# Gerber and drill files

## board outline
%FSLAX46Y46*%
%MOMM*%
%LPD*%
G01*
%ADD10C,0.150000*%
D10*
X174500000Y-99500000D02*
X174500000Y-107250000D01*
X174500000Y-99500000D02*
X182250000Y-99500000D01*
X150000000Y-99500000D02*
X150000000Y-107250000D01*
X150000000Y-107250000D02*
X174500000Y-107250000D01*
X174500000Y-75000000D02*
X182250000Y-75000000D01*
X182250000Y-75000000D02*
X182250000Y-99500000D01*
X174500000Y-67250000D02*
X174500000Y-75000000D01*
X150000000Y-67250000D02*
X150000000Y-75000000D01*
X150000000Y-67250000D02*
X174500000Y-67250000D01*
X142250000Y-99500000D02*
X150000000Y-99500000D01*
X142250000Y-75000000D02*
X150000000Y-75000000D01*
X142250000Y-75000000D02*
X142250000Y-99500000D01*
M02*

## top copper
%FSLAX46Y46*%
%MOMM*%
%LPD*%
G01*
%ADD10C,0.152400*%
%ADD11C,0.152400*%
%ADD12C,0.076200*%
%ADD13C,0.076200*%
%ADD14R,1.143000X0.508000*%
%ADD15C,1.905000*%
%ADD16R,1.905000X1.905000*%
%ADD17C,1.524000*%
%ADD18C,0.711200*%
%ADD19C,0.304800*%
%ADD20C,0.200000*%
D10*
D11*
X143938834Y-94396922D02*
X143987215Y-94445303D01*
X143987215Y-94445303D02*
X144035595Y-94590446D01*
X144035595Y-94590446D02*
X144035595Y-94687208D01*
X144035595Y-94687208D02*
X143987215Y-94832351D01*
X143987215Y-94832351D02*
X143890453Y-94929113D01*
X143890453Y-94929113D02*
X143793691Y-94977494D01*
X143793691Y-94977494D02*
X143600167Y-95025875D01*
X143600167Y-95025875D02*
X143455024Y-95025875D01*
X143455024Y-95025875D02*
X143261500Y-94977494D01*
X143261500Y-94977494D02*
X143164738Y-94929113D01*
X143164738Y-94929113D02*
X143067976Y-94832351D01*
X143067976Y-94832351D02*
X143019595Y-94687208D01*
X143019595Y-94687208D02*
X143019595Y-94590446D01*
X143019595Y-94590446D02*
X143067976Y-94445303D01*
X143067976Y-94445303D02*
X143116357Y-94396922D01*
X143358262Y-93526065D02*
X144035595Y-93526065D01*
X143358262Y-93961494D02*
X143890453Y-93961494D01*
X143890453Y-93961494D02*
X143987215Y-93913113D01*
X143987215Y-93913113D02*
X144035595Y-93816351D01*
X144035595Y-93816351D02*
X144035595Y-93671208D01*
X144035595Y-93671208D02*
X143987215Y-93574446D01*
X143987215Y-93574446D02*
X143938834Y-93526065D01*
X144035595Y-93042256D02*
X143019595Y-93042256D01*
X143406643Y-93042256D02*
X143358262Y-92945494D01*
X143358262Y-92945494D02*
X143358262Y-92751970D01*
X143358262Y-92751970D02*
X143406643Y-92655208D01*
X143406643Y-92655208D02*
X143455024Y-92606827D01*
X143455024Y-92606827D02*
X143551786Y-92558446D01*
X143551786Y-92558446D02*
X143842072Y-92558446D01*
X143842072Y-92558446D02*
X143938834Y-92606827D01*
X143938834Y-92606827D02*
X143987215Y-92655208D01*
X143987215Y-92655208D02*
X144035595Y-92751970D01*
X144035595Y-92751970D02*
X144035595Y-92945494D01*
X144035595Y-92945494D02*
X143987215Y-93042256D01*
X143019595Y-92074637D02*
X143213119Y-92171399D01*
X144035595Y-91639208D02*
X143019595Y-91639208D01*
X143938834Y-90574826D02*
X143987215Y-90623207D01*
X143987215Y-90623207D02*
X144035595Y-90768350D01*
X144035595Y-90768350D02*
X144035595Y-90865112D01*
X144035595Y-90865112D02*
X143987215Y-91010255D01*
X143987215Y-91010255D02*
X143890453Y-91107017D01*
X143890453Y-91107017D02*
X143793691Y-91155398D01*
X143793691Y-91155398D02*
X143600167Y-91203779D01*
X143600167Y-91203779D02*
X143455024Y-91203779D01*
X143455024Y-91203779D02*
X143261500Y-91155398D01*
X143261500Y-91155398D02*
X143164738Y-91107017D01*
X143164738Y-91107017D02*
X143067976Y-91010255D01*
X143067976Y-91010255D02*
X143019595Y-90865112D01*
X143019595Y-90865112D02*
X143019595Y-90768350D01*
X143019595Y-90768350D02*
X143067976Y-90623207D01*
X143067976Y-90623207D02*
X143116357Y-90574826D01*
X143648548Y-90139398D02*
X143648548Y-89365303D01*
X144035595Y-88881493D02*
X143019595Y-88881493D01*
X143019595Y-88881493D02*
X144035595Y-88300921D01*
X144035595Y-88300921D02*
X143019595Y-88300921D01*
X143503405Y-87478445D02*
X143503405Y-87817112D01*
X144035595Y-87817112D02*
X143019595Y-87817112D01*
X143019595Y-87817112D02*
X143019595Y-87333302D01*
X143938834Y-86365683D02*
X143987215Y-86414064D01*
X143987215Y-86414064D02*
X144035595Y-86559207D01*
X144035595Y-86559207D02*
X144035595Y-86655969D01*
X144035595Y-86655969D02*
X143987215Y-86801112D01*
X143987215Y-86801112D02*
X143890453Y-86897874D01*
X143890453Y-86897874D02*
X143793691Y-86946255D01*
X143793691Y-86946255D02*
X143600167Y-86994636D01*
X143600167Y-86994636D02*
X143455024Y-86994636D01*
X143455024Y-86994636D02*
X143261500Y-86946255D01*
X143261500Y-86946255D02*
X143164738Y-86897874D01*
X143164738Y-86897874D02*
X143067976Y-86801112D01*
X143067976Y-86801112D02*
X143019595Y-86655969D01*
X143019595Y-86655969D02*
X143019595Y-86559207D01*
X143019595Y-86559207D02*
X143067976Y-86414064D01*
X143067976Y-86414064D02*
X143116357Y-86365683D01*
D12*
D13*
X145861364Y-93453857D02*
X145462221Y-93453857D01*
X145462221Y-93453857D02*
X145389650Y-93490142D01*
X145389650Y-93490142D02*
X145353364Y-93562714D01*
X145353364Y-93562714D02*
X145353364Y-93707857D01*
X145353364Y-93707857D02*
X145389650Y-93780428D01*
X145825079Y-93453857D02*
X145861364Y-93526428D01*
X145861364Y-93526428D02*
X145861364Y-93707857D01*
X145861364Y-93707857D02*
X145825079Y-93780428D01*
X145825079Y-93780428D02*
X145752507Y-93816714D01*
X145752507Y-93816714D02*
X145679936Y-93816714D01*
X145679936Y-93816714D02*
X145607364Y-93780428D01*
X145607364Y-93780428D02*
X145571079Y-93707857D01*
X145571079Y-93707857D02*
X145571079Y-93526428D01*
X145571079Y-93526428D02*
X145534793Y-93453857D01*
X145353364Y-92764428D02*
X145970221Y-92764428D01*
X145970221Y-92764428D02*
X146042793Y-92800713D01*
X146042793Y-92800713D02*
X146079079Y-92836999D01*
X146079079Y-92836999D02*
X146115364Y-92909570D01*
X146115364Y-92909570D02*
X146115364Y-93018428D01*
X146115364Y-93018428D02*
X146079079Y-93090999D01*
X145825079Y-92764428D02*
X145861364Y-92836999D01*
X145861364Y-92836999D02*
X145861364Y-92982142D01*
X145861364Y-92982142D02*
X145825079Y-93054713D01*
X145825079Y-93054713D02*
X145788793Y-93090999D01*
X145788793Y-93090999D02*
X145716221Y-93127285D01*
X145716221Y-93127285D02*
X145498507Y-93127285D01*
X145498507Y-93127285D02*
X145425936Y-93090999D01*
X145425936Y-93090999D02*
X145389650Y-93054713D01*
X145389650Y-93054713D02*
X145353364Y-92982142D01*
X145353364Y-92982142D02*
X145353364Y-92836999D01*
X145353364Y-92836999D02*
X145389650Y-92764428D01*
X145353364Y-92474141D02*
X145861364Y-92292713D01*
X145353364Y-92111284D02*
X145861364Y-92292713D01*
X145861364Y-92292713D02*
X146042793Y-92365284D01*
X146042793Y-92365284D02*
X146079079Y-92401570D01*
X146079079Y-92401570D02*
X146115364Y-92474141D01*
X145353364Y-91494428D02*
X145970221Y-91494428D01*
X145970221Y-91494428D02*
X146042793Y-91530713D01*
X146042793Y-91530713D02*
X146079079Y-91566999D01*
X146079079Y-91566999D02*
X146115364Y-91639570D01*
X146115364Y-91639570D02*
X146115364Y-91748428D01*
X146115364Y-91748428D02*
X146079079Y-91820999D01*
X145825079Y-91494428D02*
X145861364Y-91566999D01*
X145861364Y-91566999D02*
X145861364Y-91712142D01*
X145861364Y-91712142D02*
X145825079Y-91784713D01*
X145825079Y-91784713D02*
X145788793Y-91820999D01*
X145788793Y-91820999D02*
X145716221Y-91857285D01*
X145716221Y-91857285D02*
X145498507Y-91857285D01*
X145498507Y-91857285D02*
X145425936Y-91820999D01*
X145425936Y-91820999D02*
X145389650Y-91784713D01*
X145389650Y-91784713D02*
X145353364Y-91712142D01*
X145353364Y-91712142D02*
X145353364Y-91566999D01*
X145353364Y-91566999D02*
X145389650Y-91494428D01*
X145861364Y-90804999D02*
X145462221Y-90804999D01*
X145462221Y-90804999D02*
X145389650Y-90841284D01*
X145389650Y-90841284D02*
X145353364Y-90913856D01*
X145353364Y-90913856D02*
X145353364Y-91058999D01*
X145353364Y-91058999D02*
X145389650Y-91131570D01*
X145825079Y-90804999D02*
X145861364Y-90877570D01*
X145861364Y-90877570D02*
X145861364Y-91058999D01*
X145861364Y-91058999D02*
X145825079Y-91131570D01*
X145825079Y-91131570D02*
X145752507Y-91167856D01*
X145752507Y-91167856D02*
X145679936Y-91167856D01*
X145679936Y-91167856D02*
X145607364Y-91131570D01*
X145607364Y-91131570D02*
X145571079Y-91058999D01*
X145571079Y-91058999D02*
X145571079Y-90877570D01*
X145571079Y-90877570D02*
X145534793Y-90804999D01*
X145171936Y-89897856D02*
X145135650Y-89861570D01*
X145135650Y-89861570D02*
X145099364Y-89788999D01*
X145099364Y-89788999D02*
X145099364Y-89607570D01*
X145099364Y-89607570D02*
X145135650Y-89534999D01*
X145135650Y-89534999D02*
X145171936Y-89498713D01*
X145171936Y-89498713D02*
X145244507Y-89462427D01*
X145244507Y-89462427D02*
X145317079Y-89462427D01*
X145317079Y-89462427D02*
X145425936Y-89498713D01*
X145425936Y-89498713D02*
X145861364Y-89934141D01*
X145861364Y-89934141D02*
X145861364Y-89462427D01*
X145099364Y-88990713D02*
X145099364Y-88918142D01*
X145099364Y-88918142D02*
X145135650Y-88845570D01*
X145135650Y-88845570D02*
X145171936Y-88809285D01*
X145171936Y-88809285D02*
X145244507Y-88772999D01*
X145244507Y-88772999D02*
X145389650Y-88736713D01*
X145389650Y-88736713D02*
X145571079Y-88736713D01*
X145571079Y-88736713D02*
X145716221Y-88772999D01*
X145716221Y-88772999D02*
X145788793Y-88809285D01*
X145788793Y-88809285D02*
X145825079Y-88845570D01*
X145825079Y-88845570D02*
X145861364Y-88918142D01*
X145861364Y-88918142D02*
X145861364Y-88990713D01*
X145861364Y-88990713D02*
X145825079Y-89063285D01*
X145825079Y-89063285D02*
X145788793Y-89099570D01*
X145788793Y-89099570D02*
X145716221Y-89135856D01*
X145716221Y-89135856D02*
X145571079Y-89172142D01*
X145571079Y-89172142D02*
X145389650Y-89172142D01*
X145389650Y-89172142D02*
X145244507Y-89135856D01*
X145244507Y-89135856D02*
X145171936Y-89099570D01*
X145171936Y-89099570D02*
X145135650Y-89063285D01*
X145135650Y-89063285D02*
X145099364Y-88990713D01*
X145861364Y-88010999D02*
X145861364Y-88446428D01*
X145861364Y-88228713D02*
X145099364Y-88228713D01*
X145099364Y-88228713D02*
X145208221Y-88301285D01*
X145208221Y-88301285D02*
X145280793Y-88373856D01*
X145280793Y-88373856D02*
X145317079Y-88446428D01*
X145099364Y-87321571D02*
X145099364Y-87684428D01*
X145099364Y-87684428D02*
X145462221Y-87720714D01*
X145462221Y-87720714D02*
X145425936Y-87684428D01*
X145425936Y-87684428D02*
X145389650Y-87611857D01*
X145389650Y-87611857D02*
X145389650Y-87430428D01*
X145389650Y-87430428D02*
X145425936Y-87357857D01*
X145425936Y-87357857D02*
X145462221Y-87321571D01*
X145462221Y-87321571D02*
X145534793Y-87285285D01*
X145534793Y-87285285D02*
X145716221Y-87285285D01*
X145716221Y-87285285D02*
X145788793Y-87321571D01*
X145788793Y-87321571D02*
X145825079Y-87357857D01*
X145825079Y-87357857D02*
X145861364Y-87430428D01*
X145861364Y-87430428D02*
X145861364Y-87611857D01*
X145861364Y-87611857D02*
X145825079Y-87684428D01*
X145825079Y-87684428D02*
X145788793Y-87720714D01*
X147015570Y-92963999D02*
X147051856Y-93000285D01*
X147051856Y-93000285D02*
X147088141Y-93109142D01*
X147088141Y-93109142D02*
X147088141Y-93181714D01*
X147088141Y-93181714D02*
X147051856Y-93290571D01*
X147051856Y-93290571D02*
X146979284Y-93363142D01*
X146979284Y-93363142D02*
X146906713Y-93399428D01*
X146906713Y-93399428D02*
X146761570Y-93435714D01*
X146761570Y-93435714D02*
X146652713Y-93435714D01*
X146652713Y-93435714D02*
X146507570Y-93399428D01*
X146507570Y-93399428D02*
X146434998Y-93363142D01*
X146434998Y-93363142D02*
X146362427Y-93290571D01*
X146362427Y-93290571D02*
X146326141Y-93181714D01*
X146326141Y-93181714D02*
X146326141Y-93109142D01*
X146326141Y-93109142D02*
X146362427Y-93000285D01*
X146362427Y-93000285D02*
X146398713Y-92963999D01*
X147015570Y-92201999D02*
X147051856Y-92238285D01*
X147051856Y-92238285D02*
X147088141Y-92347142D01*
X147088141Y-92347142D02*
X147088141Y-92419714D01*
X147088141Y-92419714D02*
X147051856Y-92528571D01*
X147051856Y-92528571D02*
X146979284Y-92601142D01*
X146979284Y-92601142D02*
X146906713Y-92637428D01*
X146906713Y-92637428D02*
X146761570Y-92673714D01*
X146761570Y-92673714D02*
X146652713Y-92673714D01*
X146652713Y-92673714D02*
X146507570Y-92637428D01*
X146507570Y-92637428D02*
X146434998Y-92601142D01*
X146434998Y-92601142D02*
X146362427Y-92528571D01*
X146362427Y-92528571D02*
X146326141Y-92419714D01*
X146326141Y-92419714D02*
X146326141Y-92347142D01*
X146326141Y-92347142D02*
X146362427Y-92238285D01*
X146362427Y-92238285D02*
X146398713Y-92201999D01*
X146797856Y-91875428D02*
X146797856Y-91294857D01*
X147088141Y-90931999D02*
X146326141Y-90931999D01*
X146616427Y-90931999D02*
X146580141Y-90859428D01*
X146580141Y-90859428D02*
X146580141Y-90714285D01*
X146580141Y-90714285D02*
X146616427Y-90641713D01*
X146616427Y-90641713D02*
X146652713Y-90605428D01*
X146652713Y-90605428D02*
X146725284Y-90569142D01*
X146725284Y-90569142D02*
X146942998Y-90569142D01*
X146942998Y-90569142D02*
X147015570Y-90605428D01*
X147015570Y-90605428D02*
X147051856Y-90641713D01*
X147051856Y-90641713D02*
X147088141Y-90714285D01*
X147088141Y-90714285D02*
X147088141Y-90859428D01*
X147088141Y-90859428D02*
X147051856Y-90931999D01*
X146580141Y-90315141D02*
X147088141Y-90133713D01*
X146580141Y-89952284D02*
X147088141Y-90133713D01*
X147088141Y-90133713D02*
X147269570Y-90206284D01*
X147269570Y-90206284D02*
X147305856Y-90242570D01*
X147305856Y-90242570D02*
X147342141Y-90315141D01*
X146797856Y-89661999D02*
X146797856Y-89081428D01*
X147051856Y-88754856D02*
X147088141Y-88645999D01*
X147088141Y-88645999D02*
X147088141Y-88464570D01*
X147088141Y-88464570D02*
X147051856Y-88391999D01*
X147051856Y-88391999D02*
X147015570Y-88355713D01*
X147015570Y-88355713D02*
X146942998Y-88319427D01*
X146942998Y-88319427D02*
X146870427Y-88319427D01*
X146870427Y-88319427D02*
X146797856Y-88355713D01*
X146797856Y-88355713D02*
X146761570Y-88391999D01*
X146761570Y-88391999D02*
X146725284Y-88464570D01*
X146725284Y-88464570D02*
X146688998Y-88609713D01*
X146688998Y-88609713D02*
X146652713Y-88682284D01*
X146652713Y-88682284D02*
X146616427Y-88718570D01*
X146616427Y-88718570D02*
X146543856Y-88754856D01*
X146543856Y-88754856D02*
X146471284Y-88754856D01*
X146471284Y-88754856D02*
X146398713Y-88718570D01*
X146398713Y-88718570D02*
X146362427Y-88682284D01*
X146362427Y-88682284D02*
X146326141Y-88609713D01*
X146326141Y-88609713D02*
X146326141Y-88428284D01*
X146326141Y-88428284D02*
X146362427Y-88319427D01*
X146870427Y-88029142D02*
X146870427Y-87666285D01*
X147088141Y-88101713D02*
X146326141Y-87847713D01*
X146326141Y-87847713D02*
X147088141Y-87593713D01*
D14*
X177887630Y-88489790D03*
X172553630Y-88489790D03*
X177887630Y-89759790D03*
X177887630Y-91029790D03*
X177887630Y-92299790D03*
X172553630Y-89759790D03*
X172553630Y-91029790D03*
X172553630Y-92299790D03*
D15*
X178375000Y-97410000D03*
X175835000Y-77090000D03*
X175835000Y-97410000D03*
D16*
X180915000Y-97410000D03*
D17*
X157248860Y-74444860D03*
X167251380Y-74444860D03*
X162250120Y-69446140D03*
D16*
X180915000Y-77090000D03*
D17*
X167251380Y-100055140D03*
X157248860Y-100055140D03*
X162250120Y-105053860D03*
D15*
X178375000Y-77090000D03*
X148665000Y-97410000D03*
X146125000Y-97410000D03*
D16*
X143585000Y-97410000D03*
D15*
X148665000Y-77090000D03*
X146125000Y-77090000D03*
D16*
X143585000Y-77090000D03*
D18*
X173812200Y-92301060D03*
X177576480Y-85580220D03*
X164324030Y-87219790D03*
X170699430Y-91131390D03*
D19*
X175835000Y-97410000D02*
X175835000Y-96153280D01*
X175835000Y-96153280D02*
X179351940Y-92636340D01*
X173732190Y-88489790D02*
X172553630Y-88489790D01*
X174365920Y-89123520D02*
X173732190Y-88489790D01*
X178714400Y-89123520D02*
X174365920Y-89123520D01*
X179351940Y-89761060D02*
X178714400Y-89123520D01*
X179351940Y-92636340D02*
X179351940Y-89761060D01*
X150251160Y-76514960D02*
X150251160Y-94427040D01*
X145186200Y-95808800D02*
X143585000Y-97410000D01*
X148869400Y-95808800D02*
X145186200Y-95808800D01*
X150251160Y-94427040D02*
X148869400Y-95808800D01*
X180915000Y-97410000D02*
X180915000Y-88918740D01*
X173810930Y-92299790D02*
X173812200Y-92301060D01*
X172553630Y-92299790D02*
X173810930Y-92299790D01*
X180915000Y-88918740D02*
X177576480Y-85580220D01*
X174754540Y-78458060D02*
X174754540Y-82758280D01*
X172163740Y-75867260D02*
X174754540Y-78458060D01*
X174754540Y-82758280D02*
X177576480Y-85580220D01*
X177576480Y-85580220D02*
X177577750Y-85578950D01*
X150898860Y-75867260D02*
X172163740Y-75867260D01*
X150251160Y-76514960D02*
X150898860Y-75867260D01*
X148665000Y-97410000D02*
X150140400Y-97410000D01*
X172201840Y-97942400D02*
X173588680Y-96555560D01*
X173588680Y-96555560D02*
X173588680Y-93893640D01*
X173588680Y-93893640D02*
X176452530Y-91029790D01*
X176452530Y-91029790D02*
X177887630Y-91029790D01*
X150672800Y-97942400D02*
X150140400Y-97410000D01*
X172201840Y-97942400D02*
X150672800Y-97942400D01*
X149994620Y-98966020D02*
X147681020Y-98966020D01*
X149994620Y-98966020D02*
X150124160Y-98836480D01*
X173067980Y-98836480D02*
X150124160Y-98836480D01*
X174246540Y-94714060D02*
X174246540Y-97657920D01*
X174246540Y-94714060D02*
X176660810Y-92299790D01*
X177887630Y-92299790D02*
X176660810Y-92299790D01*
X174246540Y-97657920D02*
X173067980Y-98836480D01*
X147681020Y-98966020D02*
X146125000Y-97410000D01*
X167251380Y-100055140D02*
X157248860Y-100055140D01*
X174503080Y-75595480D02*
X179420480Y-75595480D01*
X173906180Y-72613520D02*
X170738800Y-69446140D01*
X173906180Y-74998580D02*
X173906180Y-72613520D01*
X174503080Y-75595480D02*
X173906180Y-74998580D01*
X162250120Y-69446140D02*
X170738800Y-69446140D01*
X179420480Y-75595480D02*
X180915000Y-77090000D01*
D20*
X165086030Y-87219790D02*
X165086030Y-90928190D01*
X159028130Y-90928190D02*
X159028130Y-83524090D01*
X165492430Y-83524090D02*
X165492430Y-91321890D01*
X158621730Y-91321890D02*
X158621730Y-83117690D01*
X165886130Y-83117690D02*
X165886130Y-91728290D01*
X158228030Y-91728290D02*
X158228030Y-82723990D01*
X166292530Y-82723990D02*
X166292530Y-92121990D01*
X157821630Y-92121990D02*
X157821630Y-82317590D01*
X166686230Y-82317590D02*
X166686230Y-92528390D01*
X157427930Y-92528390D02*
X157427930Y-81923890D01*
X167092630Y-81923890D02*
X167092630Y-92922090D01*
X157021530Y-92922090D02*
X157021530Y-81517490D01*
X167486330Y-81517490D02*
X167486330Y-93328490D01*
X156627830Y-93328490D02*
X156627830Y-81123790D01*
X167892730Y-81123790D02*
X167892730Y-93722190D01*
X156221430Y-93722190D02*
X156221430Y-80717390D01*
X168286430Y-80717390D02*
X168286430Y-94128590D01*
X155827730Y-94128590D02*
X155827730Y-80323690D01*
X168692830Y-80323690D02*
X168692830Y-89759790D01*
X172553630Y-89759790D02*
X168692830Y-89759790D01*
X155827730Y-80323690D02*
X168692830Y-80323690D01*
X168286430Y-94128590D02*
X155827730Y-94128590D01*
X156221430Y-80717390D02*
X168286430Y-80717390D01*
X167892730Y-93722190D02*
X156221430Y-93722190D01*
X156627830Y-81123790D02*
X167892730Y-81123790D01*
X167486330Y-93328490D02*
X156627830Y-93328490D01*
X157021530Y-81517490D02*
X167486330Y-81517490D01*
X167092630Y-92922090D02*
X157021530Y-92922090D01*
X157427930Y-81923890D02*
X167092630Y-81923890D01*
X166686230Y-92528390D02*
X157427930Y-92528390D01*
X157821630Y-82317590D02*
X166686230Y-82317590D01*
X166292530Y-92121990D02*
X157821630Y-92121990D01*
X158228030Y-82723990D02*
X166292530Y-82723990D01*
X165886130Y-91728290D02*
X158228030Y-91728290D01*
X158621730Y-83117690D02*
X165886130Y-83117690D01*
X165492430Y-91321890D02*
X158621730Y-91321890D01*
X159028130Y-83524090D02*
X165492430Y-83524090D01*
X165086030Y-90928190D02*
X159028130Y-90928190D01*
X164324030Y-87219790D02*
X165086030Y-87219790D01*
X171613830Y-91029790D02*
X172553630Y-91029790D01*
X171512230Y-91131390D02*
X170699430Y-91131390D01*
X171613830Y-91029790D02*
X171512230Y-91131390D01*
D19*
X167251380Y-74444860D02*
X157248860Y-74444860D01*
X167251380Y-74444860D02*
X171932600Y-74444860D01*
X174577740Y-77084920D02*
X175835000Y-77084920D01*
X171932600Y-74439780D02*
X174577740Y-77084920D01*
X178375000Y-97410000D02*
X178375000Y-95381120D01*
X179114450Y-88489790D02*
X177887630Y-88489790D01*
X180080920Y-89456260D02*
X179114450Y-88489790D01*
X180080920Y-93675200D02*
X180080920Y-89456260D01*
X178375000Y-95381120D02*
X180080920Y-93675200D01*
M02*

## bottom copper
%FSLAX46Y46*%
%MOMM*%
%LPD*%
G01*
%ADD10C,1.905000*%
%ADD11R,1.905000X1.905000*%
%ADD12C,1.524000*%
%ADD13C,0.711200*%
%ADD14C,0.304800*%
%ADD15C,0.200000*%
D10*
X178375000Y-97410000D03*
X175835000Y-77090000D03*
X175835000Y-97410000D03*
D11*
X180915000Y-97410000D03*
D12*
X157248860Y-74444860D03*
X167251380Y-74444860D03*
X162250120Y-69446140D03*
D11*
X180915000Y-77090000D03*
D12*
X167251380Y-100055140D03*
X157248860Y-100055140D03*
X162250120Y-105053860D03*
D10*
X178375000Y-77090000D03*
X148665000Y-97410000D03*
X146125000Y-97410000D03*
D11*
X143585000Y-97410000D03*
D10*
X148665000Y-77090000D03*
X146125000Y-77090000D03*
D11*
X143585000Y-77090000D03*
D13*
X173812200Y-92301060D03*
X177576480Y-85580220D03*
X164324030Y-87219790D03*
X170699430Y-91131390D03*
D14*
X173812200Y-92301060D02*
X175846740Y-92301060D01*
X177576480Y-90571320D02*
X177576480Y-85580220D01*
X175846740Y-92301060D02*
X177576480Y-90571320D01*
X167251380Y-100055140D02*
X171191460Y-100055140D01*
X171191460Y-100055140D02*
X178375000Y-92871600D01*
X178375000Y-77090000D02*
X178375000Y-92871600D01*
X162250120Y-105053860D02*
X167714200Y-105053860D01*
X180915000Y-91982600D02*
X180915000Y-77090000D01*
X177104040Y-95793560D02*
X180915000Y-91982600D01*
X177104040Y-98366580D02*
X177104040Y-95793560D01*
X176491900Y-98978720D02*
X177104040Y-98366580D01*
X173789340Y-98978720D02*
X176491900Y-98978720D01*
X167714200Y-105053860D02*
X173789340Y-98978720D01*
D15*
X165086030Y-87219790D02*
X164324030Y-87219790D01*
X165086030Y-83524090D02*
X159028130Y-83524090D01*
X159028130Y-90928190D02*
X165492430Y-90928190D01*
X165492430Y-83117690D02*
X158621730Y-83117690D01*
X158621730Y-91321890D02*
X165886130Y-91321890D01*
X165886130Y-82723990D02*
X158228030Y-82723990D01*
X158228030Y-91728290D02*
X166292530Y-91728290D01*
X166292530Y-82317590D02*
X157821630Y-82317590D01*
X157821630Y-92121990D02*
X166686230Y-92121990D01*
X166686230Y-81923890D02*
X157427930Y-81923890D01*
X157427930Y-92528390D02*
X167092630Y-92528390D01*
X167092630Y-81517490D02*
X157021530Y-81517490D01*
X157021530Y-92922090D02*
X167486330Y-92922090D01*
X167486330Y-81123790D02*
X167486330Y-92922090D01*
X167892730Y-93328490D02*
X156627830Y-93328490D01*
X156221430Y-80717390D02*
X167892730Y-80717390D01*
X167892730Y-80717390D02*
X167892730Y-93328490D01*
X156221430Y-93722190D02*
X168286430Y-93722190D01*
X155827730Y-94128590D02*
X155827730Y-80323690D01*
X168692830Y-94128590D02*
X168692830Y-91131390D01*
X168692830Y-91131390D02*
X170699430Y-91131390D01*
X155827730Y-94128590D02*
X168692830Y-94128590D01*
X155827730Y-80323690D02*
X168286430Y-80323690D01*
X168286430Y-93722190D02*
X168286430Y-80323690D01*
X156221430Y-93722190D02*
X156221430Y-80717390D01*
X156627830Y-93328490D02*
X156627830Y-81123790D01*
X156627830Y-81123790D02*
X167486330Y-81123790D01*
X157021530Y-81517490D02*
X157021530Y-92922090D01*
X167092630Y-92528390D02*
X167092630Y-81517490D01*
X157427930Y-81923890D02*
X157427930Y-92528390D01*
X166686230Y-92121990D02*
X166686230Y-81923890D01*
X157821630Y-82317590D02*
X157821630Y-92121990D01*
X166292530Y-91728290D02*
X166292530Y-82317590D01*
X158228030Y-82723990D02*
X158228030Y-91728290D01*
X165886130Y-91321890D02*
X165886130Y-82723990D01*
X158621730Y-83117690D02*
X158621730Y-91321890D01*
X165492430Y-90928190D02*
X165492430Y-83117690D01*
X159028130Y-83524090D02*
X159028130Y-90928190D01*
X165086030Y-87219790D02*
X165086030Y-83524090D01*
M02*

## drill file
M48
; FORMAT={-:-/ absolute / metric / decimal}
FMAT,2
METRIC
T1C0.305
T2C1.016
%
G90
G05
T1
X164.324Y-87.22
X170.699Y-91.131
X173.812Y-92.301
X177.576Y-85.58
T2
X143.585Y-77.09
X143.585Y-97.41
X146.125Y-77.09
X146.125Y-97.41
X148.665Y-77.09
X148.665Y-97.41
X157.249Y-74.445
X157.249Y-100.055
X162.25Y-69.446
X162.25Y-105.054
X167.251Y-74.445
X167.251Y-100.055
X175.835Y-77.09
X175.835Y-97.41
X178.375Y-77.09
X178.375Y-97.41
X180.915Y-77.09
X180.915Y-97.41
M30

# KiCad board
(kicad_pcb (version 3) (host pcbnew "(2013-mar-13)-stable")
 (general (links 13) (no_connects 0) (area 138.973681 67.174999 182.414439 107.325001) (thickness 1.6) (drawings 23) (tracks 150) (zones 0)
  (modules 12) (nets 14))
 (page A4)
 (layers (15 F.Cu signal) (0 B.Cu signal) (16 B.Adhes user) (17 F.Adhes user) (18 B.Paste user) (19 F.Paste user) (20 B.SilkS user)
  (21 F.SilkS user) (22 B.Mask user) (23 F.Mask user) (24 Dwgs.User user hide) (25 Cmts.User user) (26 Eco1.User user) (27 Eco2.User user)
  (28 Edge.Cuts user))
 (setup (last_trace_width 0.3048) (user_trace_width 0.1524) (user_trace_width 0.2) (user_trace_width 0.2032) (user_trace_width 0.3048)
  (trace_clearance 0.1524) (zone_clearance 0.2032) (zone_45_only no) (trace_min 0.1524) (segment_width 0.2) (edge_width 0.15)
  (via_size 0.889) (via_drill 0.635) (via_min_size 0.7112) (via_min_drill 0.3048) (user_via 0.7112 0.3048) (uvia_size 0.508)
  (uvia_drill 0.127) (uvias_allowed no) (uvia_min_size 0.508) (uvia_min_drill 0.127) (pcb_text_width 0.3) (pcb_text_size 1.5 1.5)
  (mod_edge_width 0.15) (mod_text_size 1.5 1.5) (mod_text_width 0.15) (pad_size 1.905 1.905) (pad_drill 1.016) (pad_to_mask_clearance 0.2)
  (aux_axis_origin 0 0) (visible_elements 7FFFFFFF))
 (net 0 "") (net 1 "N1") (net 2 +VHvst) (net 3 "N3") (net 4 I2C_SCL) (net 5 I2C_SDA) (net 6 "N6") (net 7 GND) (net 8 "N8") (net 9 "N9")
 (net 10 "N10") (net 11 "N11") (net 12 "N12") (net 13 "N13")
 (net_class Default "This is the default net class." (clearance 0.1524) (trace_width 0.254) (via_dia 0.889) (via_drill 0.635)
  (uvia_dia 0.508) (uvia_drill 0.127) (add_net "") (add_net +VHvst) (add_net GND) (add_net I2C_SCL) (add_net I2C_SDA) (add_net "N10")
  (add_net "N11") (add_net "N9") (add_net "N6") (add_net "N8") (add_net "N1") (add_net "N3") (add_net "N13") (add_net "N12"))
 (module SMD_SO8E (layer F.Cu) (at 175.22063 90.39479 270)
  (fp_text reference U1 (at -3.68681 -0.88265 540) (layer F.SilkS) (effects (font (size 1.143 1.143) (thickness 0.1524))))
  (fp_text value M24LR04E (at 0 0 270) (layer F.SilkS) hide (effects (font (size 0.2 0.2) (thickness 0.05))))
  (pad 8 smd rect (at -1.905 -2.667 270) (size 0.508 1.143) (layers F.Cu F.Paste F.Mask) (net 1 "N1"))
  (pad 1 smd rect (at -1.905 2.667 270) (size 0.508 1.143) (layers F.Cu F.Paste F.Mask) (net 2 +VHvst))
  (pad 7 smd rect (at -0.635 -2.667 270) (size 0.508 1.143) (layers F.Cu F.Paste F.Mask) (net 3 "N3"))
  (pad 6 smd rect (at 0.635 -2.667 270) (size 0.508 1.143) (layers F.Cu F.Paste F.Mask) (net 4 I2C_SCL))
  (pad 5 smd rect (at 1.905 -2.667 270) (size 0.508 1.143) (layers F.Cu F.Paste F.Mask) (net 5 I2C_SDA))
  (pad 2 smd rect (at -0.635 2.667 270) (size 0.508 1.143) (layers F.Cu F.Paste F.Mask) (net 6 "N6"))
  (pad 3 smd rect (at 0.635 2.667 270) (size 0.508 1.143) (layers F.Cu F.Paste F.Mask) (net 6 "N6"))
  (pad 4 smd rect (at 1.905 2.667 270) (size 0.508 1.143) (layers F.Cu F.Paste F.Mask) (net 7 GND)))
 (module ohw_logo (layer F.Cu) (at 142.27048 78.73492)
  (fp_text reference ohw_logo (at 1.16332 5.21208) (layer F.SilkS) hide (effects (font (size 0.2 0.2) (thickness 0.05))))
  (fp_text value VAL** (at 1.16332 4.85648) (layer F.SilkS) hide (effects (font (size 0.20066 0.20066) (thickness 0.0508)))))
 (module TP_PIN (layer F.Cu) (at 178.375 97.41)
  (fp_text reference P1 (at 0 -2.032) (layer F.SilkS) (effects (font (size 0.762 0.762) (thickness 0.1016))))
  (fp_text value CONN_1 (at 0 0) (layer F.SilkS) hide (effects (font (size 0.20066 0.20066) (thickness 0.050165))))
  (pad 1 thru_hole circle (at 0 0) (size 1.905 1.905) (drill 1.016) (layers *.Cu *.Mask F.SilkS) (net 1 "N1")))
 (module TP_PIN (layer F.Cu) (at 175.835 77.09)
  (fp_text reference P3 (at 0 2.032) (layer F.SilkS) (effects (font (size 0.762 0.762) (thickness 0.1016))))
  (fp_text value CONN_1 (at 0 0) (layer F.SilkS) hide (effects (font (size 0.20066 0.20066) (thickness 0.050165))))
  (pad 1 thru_hole circle (at 0 0) (size 1.905 1.905) (drill 1.016) (layers *.Cu *.Mask F.SilkS) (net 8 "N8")))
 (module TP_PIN (layer F.Cu) (at 175.835 97.41)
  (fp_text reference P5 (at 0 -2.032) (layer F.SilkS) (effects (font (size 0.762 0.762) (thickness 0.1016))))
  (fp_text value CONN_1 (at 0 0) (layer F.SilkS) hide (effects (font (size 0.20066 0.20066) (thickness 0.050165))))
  (pad 1 thru_hole circle (at 0 0) (size 1.905 1.905) (drill 1.016) (layers *.Cu *.Mask F.SilkS) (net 2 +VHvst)))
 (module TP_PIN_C (layer F.Cu) (at 180.915 97.41)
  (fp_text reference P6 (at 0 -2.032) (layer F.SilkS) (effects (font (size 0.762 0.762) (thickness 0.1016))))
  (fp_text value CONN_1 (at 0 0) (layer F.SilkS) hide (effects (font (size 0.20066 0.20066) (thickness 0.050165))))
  (pad 1 thru_hole rect (at 0 0) (size 1.905 1.905) (drill 1.016) (layers *.Cu *.Mask F.SilkS) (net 7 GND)))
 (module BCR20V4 (layer F.Cu) (at 162.25012 71.9455)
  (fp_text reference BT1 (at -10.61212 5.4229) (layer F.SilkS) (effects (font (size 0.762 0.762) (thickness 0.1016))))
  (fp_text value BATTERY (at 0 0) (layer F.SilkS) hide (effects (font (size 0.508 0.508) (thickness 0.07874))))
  (pad 1 thru_hole circle (at -5.00126 2.49936) (size 1.524 1.524) (drill 1.016) (layers *.Cu *.Mask) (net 8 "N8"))
  (pad 1 thru_hole circle (at 5.00126 2.49936) (size 1.524 1.524) (drill 1.016) (layers *.Cu *.Mask) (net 8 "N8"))
  (pad 2 thru_hole circle (at 0 -2.49936) (size 1.524 1.524) (drill 1.016) (layers *.Cu *.Mask) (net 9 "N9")))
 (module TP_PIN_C (layer F.Cu) (at 180.915 77.09)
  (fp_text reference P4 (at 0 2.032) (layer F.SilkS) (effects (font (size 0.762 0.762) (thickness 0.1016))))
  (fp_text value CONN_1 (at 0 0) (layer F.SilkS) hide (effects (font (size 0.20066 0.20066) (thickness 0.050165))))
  (pad 1 thru_hole rect (at 0 0) (size 1.905 1.905) (drill 1.016) (layers *.Cu *.Mask F.SilkS) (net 9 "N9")))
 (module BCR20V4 (layer F.Cu) (at 162.25012 102.5545 180)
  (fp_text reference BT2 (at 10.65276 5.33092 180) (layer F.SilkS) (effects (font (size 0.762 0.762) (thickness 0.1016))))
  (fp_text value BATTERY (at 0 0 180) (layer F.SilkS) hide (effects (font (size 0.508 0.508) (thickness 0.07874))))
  (pad 1 thru_hole circle (at -5.00126 2.49936 180) (size 1.524 1.524) (drill 1.016) (layers *.Cu *.Mask) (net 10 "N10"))
  (pad 1 thru_hole circle (at 5.00126 2.49936 180) (size 1.524 1.524) (drill 1.016) (layers *.Cu *.Mask) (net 10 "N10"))
  (pad 2 thru_hole circle (at 0 -2.49936 180) (size 1.524 1.524) (drill 1.016) (layers *.Cu *.Mask) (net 9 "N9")))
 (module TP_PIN (layer F.Cu) (at 178.375 77.09)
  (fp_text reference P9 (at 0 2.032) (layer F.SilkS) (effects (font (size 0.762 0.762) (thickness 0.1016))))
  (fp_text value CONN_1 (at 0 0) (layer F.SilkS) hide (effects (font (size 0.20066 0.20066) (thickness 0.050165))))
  (pad 1 thru_hole circle (at 0 0) (size 1.905 1.905) (drill 1.016) (layers *.Cu *.Mask F.SilkS) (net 10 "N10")))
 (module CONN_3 (layer F.Cu) (at 146.125 97.41)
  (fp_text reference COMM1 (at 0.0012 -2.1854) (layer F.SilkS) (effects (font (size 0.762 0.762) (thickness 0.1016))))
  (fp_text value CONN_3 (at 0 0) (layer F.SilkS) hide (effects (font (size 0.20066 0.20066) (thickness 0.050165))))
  (pad 3 thru_hole circle (at 2.54 0) (size 1.905 1.905) (drill 1.016) (layers *.Cu *.Mask F.SilkS) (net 4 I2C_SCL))
  (pad 2 thru_hole circle (at 0 0) (size 1.905 1.905) (drill 1.016) (layers *.Cu *.Mask F.SilkS) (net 5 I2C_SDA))
  (pad 1 thru_hole rect (at -2.54 0) (size 1.905 1.905) (drill 1.016) (layers *.Cu *.Mask F.SilkS) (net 7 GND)))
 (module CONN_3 (layer F.Cu) (at 146.125 77.09)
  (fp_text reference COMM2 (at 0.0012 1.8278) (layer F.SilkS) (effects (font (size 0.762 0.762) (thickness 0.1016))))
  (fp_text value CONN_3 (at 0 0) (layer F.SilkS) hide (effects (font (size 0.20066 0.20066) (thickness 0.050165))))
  (pad 3 thru_hole circle (at 2.54 0) (size 1.905 1.905) (drill 1.016) (layers *.Cu *.Mask F.SilkS) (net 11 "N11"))
  (pad 2 thru_hole circle (at 0 0) (size 1.905 1.905) (drill 1.016) (layers *.Cu *.Mask F.SilkS) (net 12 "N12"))
  (pad 1 thru_hole rect (at -2.54 0) (size 1.905 1.905) (drill 1.016) (layers *.Cu *.Mask F.SilkS) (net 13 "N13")))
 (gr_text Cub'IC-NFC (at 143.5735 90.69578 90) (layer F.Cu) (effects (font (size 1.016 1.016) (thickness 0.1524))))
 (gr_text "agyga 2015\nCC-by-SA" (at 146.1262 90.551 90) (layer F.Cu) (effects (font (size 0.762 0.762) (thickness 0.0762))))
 (gr_line (start 174.5 99.5) (end 174.5 107.25) (angle 90) (layer Edge.Cuts) (width 0.15))
 (gr_line (start 174.5 99.5) (end 182.25 99.5) (angle 90) (layer Edge.Cuts) (width 0.15))
 (gr_line (start 150 99.5) (end 150 107.25) (angle 90) (layer Edge.Cuts) (width 0.15))
 (gr_line (start 150 107.25) (end 174.5 107.25) (angle 90) (layer Edge.Cuts) (width 0.15))
 (gr_line (start 174.5 75) (end 182.25 75) (angle 90) (layer Edge.Cuts) (width 0.15))
 (gr_line (start 182.25 75) (end 182.25 99.5) (angle 90) (layer Edge.Cuts) (width 0.15))
 (gr_line (start 174.5 67.25) (end 174.5 75) (angle 90) (layer Edge.Cuts) (width 0.15))
 (gr_line (start 150 67.25) (end 150 75) (angle 90) (layer Edge.Cuts) (width 0.15))
 (gr_line (start 150 67.25) (end 174.5 67.25) (angle 90) (layer Edge.Cuts) (width 0.15))
 (gr_line (start 142.25 99.5) (end 150 99.5) (angle 90) (layer Edge.Cuts) (width 0.15))
 (gr_line (start 142.25 75) (end 150 75) (angle 90) (layer Edge.Cuts) (width 0.15))
 (gr_line (start 142.25 75) (end 142.25 99.5) (angle 90) (layer Edge.Cuts) (width 0.15))
 (segment (start 175.835 97.41) (end 175.835 96.15328) (width 0.3048) (layer F.Cu) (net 2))
 (segment (start 175.835 96.15328) (end 179.35194 92.63634) (width 0.3048) (layer F.Cu) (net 2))
 (segment (start 173.73219 88.48979) (end 172.55363 88.48979) (width 0.3048) (layer F.Cu) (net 2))
 (segment (start 174.36592 89.12352) (end 173.73219 88.48979) (width 0.3048) (layer F.Cu) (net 2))
 (segment (start 178.7144 89.12352) (end 174.36592 89.12352) (width 0.3048) (layer F.Cu) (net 2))
 (segment (start 179.35194 89.76106) (end 178.7144 89.12352) (width 0.3048) (layer F.Cu) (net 2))
 (segment (start 179.35194 92.63634) (end 179.35194 89.76106) (width 0.3048) (layer F.Cu) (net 2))
 (segment (start 150.25116 76.51496) (end 150.25116 94.42704) (width 0.3048) (layer F.Cu) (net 7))
 (segment (start 145.1862 95.8088) (end 143.585 97.41) (width 0.3048) (layer F.Cu) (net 7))
 (segment (start 148.8694 95.8088) (end 145.1862 95.8088) (width 0.3048) (layer F.Cu) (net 7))
 (segment (start 150.25116 94.42704) (end 148.8694 95.8088) (width 0.3048) (layer F.Cu) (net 7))
 (segment (start 180.915 97.41) (end 180.915 88.91874) (width 0.3048) (layer F.Cu) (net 7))
 (segment (start 173.8122 92.30106) (end 175.84674 92.30106) (width 0.3048) (layer B.Cu) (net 7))
 (segment (start 173.81093 92.29979) (end 173.8122 92.30106) (width 0.3048) (layer F.Cu) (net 7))
 (via (at 173.8122 92.30106) (size 0.7112) (drill 0.3048) (layers F.Cu B.Cu) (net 7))
 (segment (start 172.55363 92.29979) (end 173.81093 92.29979) (width 0.3048) (layer F.Cu) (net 7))
 (segment (start 180.915 88.91874) (end 177.57648 85.58022) (width 0.3048) (layer F.Cu) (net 7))
 (segment (start 174.75454 78.45806) (end 174.75454 82.75828) (width 0.3048) (layer F.Cu) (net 7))
 (segment (start 172.16374 75.86726) (end 174.75454 78.45806) (width 0.3048) (layer F.Cu) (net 7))
 (segment (start 174.75454 82.75828) (end 177.57648 85.58022) (width 0.3048) (layer F.Cu) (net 7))
 (segment (start 177.57648 85.58022) (end 177.57775 85.57895) (width 0.3048) (layer F.Cu) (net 7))
 (via (at 177.57648 85.58022) (size 0.7112) (drill 0.3048) (layers F.Cu B.Cu) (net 7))
 (segment (start 177.57648 90.57132) (end 177.57648 85.58022) (width 0.3048) (layer B.Cu) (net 7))
 (segment (start 175.84674 92.30106) (end 177.57648 90.57132) (width 0.3048) (layer B.Cu) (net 7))
 (segment (start 150.89886 75.86726) (end 172.16374 75.86726) (width 0.3048) (layer F.Cu) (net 7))
 (segment (start 150.25116 76.51496) (end 150.89886 75.86726) (width 0.3048) (layer F.Cu) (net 7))
 (segment (start 148.665 97.41) (end 150.1404 97.41) (width 0.3048) (layer F.Cu) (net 4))
 (segment (start 172.20184 97.9424) (end 173.58868 96.55556) (width 0.3048) (layer F.Cu) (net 4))
 (segment (start 173.58868 96.55556) (end 173.58868 93.89364) (width 0.3048) (layer F.Cu) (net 4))
 (segment (start 173.58868 93.89364) (end 176.45253 91.02979) (width 0.3048) (layer F.Cu) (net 4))
 (segment (start 176.45253 91.02979) (end 177.88763 91.02979) (width 0.3048) (layer F.Cu) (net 4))
 (segment (start 150.6728 97.9424) (end 150.1404 97.41) (width 0.3048) (layer F.Cu) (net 4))
 (segment (start 172.20184 97.9424) (end 150.6728 97.9424) (width 0.3048) (layer F.Cu) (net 4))
 (segment (start 149.99462 98.96602) (end 147.68102 98.96602) (width 0.3048) (layer F.Cu) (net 5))
 (segment (start 149.99462 98.96602) (end 150.12416 98.83648) (width 0.3048) (layer F.Cu) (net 5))
 (segment (start 173.06798 98.83648) (end 150.12416 98.83648) (width 0.3048) (layer F.Cu) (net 5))
 (segment (start 174.24654 94.71406) (end 174.24654 97.65792) (width 0.3048) (layer F.Cu) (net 5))
 (segment (start 174.24654 94.71406) (end 176.66081 92.29979) (width 0.3048) (layer F.Cu) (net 5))
 (segment (start 177.88763 92.29979) (end 176.66081 92.29979) (width 0.3048) (layer F.Cu) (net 5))
 (segment (start 174.24654 97.65792) (end 173.06798 98.83648) (width 0.3048) (layer F.Cu) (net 5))
 (segment (start 147.68102 98.96602) (end 146.125 97.41) (width 0.3048) (layer F.Cu) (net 5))
 (segment (start 167.25138 100.05514) (end 171.19146 100.05514) (width 0.3048) (layer B.Cu) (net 10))
 (segment (start 171.19146 100.05514) (end 178.375 92.8716) (width 0.3048) (layer B.Cu) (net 10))
 (segment (start 167.25138 100.05514) (end 157.24886 100.05514) (width 0.3048) (layer F.Cu) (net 10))
 (segment (start 178.375 77.09) (end 178.375 92.8716) (width 0.3048) (layer B.Cu) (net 10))
 (segment (start 162.25012 105.05386) (end 167.7142 105.05386) (width 0.3048) (layer B.Cu) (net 9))
 (segment (start 180.915 91.9826) (end 180.915 77.09) (width 0.3048) (layer B.Cu) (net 9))
 (segment (start 177.10404 95.79356) (end 180.915 91.9826) (width 0.3048) (layer B.Cu) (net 9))
 (segment (start 177.10404 98.36658) (end 177.10404 95.79356) (width 0.3048) (layer B.Cu) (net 9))
 (segment (start 176.4919 98.97872) (end 177.10404 98.36658) (width 0.3048) (layer B.Cu) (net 9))
 (segment (start 173.78934 98.97872) (end 176.4919 98.97872) (width 0.3048) (layer B.Cu) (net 9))
 (segment (start 167.7142 105.05386) (end 173.78934 98.97872) (width 0.3048) (layer B.Cu) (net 9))
 (segment (start 174.50308 75.59548) (end 179.42048 75.59548) (width 0.3048) (layer F.Cu) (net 9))
 (segment (start 173.90618 72.61352) (end 170.7388 69.44614) (width 0.3048) (layer F.Cu) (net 9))
 (segment (start 173.90618 74.99858) (end 173.90618 72.61352) (width 0.3048) (layer F.Cu) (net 9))
 (segment (start 174.50308 75.59548) (end 173.90618 74.99858) (width 0.3048) (layer F.Cu) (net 9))
 (segment (start 162.25012 69.44614) (end 170.7388 69.44614) (width 0.3048) (layer F.Cu) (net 9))
 (segment (start 179.42048 75.59548) (end 180.915 77.09) (width 0.3048) (layer F.Cu) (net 9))
 (segment (start 165.08603 87.21979) (end 164.32403 87.21979) (width 0.2) (layer B.Cu) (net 6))
 (via (at 164.32403 87.21979) (size 0.7112) (drill 0.3048) (layers F.Cu B.Cu) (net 6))
 (segment (start 165.08603 87.21979) (end 165.08603 90.92819) (width 0.2) (layer F.Cu) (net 6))
 (segment (start 159.02813 90.92819) (end 159.02813 83.52409) (width 0.2) (layer F.Cu) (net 6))
 (segment (start 165.49243 83.52409) (end 165.49243 91.32189) (width 0.2) (layer F.Cu) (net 6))
 (segment (start 158.62173 91.32189) (end 158.62173 83.11769) (width 0.2) (layer F.Cu) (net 6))
 (segment (start 165.88613 83.11769) (end 165.88613 91.72829) (width 0.2) (layer F.Cu) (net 6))
 (segment (start 158.22803 91.72829) (end 158.22803 82.72399) (width 0.2) (layer F.Cu) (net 6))
 (segment (start 166.29253 82.72399) (end 166.29253 92.12199) (width 0.2) (layer F.Cu) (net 6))
 (segment (start 157.82163 92.12199) (end 157.82163 82.31759) (width 0.2) (layer F.Cu) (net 6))
 (segment (start 166.68623 82.31759) (end 166.68623 92.52839) (width 0.2) (layer F.Cu) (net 6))
 (segment (start 157.42793 92.52839) (end 157.42793 81.92389) (width 0.2) (layer F.Cu) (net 6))
 (segment (start 167.09263 81.92389) (end 167.09263 92.92209) (width 0.2) (layer F.Cu) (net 6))
 (segment (start 157.02153 92.92209) (end 157.02153 81.51749) (width 0.2) (layer F.Cu) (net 6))
 (segment (start 167.48633 81.51749) (end 167.48633 93.32849) (width 0.2) (layer F.Cu) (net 6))
 (segment (start 156.62783 93.32849) (end 156.62783 81.12379) (width 0.2) (layer F.Cu) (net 6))
 (segment (start 167.89273 81.12379) (end 167.89273 93.72219) (width 0.2) (layer F.Cu) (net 6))
 (segment (start 156.22143 93.72219) (end 156.22143 80.71739) (width 0.2) (layer F.Cu) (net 6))
 (segment (start 168.28643 80.71739) (end 168.28643 94.12859) (width 0.2) (layer F.Cu) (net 6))
 (segment (start 155.82773 94.12859) (end 155.82773 80.32369) (width 0.2) (layer F.Cu) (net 6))
 (segment (start 168.69283 80.32369) (end 168.69283 89.75979) (width 0.2) (layer F.Cu) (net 6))
 (segment (start 172.55363 89.75979) (end 168.69283 89.75979) (width 0.2) (layer F.Cu) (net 6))
 (segment (start 155.82773 80.32369) (end 168.69283 80.32369) (width 0.2) (layer F.Cu) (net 6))
 (segment (start 168.28643 94.12859) (end 155.82773 94.12859) (width 0.2) (layer F.Cu) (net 6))
 (segment (start 156.22143 80.71739) (end 168.28643 80.71739) (width 0.2) (layer F.Cu) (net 6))
 (segment (start 167.89273 93.72219) (end 156.22143 93.72219) (width 0.2) (layer F.Cu) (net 6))
 (segment (start 156.62783 81.12379) (end 167.89273 81.12379) (width 0.2) (layer F.Cu) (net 6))
 (segment (start 167.48633 93.32849) (end 156.62783 93.32849) (width 0.2) (layer F.Cu) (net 6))
 (segment (start 157.02153 81.51749) (end 167.48633 81.51749) (width 0.2) (layer F.Cu) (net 6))
 (segment (start 167.09263 92.92209) (end 157.02153 92.92209) (width 0.2) (layer F.Cu) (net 6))
 (segment (start 157.42793 81.92389) (end 167.09263 81.92389) (width 0.2) (layer F.Cu) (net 6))
 (segment (start 166.68623 92.52839) (end 157.42793 92.52839) (width 0.2) (layer F.Cu) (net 6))
 (segment (start 157.82163 82.31759) (end 166.68623 82.31759) (width 0.2) (layer F.Cu) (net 6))
 (segment (start 166.29253 92.12199) (end 157.82163 92.12199) (width 0.2) (layer F.Cu) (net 6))
 (segment (start 158.22803 82.72399) (end 166.29253 82.72399) (width 0.2) (layer F.Cu) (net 6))
 (segment (start 165.88613 91.72829) (end 158.22803 91.72829) (width 0.2) (layer F.Cu) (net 6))
 (segment (start 158.62173 83.11769) (end 165.88613 83.11769) (width 0.2) (layer F.Cu) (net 6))
 (segment (start 165.49243 91.32189) (end 158.62173 91.32189) (width 0.2) (layer F.Cu) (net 6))
 (segment (start 159.02813 83.52409) (end 165.49243 83.52409) (width 0.2) (layer F.Cu) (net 6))
 (segment (start 165.08603 90.92819) (end 159.02813 90.92819) (width 0.2) (layer F.Cu) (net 6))
 (segment (start 164.32403 87.21979) (end 165.08603 87.21979) (width 0.2) (layer F.Cu) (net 6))
 (segment (start 165.08603 83.52409) (end 159.02813 83.52409) (width 0.2) (layer B.Cu) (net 6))
 (segment (start 159.02813 90.92819) (end 165.49243 90.92819) (width 0.2) (layer B.Cu) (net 6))
 (segment (start 165.49243 83.11769) (end 158.62173 83.11769) (width 0.2) (layer B.Cu) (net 6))
 (segment (start 158.62173 91.32189) (end 165.88613 91.32189) (width 0.2) (layer B.Cu) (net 6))
 (segment (start 165.88613 82.72399) (end 158.22803 82.72399) (width 0.2) (layer B.Cu) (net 6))
 (segment (start 158.22803 91.72829) (end 166.29253 91.72829) (width 0.2) (layer B.Cu) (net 6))
 (segment (start 166.29253 82.31759) (end 157.82163 82.31759) (width 0.2) (layer B.Cu) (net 6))
 (segment (start 157.82163 92.12199) (end 166.68623 92.12199) (width 0.2) (layer B.Cu) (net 6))
 (segment (start 166.68623 81.92389) (end 157.42793 81.92389) (width 0.2) (layer B.Cu) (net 6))
 (segment (start 157.42793 92.52839) (end 167.09263 92.52839) (width 0.2) (layer B.Cu) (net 6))
 (segment (start 167.09263 81.51749) (end 157.02153 81.51749) (width 0.2) (layer B.Cu) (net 6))
 (segment (start 157.02153 92.92209) (end 167.48633 92.92209) (width 0.2) (layer B.Cu) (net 6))
 (segment (start 167.48633 81.12379) (end 167.48633 92.92209) (width 0.2) (layer B.Cu) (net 6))
 (segment (start 167.89273 93.32849) (end 156.62783 93.32849) (width 0.2) (layer B.Cu) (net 6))
 (segment (start 156.22143 80.71739) (end 167.89273 80.71739) (width 0.2) (layer B.Cu) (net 6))
 (segment (start 167.89273 80.71739) (end 167.89273 93.32849) (width 0.2) (layer B.Cu) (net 6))
 (segment (start 156.22143 93.72219) (end 168.28643 93.72219) (width 0.2) (layer B.Cu) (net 6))
 (segment (start 155.82773 94.12859) (end 155.82773 80.32369) (width 0.2) (layer B.Cu) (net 6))
 (segment (start 168.69283 94.12859) (end 168.69283 91.13139) (width 0.2) (layer B.Cu) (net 6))
 (segment (start 171.61383 91.02979) (end 172.55363 91.02979) (width 0.2) (layer F.Cu) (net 6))
 (via (at 170.69943 91.13139) (size 0.7112) (drill 0.3048) (layers F.Cu B.Cu) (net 6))
 (segment (start 171.51223 91.13139) (end 170.69943 91.13139) (width 0.2) (layer F.Cu) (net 6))
 (segment (start 171.61383 91.02979) (end 171.51223 91.13139) (width 0.2) (layer F.Cu) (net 6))
 (segment (start 168.69283 91.13139) (end 170.69943 91.13139) (width 0.2) (layer B.Cu) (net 6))
 (segment (start 155.82773 94.12859) (end 168.69283 94.12859) (width 0.2) (layer B.Cu) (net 6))
 (segment (start 155.82773 80.32369) (end 168.28643 80.32369) (width 0.2) (layer B.Cu) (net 6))
 (segment (start 168.28643 93.72219) (end 168.28643 80.32369) (width 0.2) (layer B.Cu) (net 6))
 (segment (start 156.22143 93.72219) (end 156.22143 80.71739) (width 0.2) (layer B.Cu) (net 6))
 (segment (start 156.62783 93.32849) (end 156.62783 81.12379) (width 0.2) (layer B.Cu) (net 6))
 (segment (start 156.62783 81.12379) (end 167.48633 81.12379) (width 0.2) (layer B.Cu) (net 6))
 (segment (start 157.02153 81.51749) (end 157.02153 92.92209) (width 0.2) (layer B.Cu) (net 6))
 (segment (start 167.09263 92.52839) (end 167.09263 81.51749) (width 0.2) (layer B.Cu) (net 6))
 (segment (start 157.42793 81.92389) (end 157.42793 92.52839) (width 0.2) (layer B.Cu) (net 6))
 (segment (start 166.68623 92.12199) (end 166.68623 81.92389) (width 0.2) (layer B.Cu) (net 6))
 (segment (start 157.82163 82.31759) (end 157.82163 92.12199) (width 0.2) (layer B.Cu) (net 6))
 (segment (start 166.29253 91.72829) (end 166.29253 82.31759) (width 0.2) (layer B.Cu) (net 6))
 (segment (start 158.22803 82.72399) (end 158.22803 91.72829) (width 0.2) (layer B.Cu) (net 6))
 (segment (start 165.88613 91.32189) (end 165.88613 82.72399) (width 0.2) (layer B.Cu) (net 6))
 (segment (start 158.62173 83.11769) (end 158.62173 91.32189) (width 0.2) (layer B.Cu) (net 6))
 (segment (start 165.49243 90.92819) (end 165.49243 83.11769) (width 0.2) (layer B.Cu) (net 6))
 (segment (start 159.02813 83.52409) (end 159.02813 90.92819) (width 0.2) (layer B.Cu) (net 6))
 (segment (start 165.08603 87.21979) (end 165.08603 83.52409) (width 0.2) (layer B.Cu) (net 6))
 (segment (start 167.25138 74.44486) (end 157.24886 74.44486) (width 0.3048) (layer F.Cu) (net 8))
 (segment (start 167.25138 74.44486) (end 171.9326 74.44486) (width 0.3048) (layer F.Cu) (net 8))
 (segment (start 174.57774 77.08492) (end 175.835 77.08492) (width 0.3048) (layer F.Cu) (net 8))
 (segment (start 171.9326 74.43978) (end 174.57774 77.08492) (width 0.3048) (layer F.Cu) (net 8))
 (segment (start 178.375 97.41) (end 178.375 95.38112) (width 0.3048) (layer F.Cu) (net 1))
 (segment (start 179.11445 88.48979) (end 177.88763 88.48979) (width 0.3048) (layer F.Cu) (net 1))
 (segment (start 180.08092 89.45626) (end 179.11445 88.48979) (width 0.3048) (layer F.Cu) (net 1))
 (segment (start 180.08092 93.6752) (end 180.08092 89.45626) (width 0.3048) (layer F.Cu) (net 1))
 (segment (start 178.375 95.38112) (end 180.08092 93.6752) (width 0.3048) (layer F.Cu) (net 1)))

